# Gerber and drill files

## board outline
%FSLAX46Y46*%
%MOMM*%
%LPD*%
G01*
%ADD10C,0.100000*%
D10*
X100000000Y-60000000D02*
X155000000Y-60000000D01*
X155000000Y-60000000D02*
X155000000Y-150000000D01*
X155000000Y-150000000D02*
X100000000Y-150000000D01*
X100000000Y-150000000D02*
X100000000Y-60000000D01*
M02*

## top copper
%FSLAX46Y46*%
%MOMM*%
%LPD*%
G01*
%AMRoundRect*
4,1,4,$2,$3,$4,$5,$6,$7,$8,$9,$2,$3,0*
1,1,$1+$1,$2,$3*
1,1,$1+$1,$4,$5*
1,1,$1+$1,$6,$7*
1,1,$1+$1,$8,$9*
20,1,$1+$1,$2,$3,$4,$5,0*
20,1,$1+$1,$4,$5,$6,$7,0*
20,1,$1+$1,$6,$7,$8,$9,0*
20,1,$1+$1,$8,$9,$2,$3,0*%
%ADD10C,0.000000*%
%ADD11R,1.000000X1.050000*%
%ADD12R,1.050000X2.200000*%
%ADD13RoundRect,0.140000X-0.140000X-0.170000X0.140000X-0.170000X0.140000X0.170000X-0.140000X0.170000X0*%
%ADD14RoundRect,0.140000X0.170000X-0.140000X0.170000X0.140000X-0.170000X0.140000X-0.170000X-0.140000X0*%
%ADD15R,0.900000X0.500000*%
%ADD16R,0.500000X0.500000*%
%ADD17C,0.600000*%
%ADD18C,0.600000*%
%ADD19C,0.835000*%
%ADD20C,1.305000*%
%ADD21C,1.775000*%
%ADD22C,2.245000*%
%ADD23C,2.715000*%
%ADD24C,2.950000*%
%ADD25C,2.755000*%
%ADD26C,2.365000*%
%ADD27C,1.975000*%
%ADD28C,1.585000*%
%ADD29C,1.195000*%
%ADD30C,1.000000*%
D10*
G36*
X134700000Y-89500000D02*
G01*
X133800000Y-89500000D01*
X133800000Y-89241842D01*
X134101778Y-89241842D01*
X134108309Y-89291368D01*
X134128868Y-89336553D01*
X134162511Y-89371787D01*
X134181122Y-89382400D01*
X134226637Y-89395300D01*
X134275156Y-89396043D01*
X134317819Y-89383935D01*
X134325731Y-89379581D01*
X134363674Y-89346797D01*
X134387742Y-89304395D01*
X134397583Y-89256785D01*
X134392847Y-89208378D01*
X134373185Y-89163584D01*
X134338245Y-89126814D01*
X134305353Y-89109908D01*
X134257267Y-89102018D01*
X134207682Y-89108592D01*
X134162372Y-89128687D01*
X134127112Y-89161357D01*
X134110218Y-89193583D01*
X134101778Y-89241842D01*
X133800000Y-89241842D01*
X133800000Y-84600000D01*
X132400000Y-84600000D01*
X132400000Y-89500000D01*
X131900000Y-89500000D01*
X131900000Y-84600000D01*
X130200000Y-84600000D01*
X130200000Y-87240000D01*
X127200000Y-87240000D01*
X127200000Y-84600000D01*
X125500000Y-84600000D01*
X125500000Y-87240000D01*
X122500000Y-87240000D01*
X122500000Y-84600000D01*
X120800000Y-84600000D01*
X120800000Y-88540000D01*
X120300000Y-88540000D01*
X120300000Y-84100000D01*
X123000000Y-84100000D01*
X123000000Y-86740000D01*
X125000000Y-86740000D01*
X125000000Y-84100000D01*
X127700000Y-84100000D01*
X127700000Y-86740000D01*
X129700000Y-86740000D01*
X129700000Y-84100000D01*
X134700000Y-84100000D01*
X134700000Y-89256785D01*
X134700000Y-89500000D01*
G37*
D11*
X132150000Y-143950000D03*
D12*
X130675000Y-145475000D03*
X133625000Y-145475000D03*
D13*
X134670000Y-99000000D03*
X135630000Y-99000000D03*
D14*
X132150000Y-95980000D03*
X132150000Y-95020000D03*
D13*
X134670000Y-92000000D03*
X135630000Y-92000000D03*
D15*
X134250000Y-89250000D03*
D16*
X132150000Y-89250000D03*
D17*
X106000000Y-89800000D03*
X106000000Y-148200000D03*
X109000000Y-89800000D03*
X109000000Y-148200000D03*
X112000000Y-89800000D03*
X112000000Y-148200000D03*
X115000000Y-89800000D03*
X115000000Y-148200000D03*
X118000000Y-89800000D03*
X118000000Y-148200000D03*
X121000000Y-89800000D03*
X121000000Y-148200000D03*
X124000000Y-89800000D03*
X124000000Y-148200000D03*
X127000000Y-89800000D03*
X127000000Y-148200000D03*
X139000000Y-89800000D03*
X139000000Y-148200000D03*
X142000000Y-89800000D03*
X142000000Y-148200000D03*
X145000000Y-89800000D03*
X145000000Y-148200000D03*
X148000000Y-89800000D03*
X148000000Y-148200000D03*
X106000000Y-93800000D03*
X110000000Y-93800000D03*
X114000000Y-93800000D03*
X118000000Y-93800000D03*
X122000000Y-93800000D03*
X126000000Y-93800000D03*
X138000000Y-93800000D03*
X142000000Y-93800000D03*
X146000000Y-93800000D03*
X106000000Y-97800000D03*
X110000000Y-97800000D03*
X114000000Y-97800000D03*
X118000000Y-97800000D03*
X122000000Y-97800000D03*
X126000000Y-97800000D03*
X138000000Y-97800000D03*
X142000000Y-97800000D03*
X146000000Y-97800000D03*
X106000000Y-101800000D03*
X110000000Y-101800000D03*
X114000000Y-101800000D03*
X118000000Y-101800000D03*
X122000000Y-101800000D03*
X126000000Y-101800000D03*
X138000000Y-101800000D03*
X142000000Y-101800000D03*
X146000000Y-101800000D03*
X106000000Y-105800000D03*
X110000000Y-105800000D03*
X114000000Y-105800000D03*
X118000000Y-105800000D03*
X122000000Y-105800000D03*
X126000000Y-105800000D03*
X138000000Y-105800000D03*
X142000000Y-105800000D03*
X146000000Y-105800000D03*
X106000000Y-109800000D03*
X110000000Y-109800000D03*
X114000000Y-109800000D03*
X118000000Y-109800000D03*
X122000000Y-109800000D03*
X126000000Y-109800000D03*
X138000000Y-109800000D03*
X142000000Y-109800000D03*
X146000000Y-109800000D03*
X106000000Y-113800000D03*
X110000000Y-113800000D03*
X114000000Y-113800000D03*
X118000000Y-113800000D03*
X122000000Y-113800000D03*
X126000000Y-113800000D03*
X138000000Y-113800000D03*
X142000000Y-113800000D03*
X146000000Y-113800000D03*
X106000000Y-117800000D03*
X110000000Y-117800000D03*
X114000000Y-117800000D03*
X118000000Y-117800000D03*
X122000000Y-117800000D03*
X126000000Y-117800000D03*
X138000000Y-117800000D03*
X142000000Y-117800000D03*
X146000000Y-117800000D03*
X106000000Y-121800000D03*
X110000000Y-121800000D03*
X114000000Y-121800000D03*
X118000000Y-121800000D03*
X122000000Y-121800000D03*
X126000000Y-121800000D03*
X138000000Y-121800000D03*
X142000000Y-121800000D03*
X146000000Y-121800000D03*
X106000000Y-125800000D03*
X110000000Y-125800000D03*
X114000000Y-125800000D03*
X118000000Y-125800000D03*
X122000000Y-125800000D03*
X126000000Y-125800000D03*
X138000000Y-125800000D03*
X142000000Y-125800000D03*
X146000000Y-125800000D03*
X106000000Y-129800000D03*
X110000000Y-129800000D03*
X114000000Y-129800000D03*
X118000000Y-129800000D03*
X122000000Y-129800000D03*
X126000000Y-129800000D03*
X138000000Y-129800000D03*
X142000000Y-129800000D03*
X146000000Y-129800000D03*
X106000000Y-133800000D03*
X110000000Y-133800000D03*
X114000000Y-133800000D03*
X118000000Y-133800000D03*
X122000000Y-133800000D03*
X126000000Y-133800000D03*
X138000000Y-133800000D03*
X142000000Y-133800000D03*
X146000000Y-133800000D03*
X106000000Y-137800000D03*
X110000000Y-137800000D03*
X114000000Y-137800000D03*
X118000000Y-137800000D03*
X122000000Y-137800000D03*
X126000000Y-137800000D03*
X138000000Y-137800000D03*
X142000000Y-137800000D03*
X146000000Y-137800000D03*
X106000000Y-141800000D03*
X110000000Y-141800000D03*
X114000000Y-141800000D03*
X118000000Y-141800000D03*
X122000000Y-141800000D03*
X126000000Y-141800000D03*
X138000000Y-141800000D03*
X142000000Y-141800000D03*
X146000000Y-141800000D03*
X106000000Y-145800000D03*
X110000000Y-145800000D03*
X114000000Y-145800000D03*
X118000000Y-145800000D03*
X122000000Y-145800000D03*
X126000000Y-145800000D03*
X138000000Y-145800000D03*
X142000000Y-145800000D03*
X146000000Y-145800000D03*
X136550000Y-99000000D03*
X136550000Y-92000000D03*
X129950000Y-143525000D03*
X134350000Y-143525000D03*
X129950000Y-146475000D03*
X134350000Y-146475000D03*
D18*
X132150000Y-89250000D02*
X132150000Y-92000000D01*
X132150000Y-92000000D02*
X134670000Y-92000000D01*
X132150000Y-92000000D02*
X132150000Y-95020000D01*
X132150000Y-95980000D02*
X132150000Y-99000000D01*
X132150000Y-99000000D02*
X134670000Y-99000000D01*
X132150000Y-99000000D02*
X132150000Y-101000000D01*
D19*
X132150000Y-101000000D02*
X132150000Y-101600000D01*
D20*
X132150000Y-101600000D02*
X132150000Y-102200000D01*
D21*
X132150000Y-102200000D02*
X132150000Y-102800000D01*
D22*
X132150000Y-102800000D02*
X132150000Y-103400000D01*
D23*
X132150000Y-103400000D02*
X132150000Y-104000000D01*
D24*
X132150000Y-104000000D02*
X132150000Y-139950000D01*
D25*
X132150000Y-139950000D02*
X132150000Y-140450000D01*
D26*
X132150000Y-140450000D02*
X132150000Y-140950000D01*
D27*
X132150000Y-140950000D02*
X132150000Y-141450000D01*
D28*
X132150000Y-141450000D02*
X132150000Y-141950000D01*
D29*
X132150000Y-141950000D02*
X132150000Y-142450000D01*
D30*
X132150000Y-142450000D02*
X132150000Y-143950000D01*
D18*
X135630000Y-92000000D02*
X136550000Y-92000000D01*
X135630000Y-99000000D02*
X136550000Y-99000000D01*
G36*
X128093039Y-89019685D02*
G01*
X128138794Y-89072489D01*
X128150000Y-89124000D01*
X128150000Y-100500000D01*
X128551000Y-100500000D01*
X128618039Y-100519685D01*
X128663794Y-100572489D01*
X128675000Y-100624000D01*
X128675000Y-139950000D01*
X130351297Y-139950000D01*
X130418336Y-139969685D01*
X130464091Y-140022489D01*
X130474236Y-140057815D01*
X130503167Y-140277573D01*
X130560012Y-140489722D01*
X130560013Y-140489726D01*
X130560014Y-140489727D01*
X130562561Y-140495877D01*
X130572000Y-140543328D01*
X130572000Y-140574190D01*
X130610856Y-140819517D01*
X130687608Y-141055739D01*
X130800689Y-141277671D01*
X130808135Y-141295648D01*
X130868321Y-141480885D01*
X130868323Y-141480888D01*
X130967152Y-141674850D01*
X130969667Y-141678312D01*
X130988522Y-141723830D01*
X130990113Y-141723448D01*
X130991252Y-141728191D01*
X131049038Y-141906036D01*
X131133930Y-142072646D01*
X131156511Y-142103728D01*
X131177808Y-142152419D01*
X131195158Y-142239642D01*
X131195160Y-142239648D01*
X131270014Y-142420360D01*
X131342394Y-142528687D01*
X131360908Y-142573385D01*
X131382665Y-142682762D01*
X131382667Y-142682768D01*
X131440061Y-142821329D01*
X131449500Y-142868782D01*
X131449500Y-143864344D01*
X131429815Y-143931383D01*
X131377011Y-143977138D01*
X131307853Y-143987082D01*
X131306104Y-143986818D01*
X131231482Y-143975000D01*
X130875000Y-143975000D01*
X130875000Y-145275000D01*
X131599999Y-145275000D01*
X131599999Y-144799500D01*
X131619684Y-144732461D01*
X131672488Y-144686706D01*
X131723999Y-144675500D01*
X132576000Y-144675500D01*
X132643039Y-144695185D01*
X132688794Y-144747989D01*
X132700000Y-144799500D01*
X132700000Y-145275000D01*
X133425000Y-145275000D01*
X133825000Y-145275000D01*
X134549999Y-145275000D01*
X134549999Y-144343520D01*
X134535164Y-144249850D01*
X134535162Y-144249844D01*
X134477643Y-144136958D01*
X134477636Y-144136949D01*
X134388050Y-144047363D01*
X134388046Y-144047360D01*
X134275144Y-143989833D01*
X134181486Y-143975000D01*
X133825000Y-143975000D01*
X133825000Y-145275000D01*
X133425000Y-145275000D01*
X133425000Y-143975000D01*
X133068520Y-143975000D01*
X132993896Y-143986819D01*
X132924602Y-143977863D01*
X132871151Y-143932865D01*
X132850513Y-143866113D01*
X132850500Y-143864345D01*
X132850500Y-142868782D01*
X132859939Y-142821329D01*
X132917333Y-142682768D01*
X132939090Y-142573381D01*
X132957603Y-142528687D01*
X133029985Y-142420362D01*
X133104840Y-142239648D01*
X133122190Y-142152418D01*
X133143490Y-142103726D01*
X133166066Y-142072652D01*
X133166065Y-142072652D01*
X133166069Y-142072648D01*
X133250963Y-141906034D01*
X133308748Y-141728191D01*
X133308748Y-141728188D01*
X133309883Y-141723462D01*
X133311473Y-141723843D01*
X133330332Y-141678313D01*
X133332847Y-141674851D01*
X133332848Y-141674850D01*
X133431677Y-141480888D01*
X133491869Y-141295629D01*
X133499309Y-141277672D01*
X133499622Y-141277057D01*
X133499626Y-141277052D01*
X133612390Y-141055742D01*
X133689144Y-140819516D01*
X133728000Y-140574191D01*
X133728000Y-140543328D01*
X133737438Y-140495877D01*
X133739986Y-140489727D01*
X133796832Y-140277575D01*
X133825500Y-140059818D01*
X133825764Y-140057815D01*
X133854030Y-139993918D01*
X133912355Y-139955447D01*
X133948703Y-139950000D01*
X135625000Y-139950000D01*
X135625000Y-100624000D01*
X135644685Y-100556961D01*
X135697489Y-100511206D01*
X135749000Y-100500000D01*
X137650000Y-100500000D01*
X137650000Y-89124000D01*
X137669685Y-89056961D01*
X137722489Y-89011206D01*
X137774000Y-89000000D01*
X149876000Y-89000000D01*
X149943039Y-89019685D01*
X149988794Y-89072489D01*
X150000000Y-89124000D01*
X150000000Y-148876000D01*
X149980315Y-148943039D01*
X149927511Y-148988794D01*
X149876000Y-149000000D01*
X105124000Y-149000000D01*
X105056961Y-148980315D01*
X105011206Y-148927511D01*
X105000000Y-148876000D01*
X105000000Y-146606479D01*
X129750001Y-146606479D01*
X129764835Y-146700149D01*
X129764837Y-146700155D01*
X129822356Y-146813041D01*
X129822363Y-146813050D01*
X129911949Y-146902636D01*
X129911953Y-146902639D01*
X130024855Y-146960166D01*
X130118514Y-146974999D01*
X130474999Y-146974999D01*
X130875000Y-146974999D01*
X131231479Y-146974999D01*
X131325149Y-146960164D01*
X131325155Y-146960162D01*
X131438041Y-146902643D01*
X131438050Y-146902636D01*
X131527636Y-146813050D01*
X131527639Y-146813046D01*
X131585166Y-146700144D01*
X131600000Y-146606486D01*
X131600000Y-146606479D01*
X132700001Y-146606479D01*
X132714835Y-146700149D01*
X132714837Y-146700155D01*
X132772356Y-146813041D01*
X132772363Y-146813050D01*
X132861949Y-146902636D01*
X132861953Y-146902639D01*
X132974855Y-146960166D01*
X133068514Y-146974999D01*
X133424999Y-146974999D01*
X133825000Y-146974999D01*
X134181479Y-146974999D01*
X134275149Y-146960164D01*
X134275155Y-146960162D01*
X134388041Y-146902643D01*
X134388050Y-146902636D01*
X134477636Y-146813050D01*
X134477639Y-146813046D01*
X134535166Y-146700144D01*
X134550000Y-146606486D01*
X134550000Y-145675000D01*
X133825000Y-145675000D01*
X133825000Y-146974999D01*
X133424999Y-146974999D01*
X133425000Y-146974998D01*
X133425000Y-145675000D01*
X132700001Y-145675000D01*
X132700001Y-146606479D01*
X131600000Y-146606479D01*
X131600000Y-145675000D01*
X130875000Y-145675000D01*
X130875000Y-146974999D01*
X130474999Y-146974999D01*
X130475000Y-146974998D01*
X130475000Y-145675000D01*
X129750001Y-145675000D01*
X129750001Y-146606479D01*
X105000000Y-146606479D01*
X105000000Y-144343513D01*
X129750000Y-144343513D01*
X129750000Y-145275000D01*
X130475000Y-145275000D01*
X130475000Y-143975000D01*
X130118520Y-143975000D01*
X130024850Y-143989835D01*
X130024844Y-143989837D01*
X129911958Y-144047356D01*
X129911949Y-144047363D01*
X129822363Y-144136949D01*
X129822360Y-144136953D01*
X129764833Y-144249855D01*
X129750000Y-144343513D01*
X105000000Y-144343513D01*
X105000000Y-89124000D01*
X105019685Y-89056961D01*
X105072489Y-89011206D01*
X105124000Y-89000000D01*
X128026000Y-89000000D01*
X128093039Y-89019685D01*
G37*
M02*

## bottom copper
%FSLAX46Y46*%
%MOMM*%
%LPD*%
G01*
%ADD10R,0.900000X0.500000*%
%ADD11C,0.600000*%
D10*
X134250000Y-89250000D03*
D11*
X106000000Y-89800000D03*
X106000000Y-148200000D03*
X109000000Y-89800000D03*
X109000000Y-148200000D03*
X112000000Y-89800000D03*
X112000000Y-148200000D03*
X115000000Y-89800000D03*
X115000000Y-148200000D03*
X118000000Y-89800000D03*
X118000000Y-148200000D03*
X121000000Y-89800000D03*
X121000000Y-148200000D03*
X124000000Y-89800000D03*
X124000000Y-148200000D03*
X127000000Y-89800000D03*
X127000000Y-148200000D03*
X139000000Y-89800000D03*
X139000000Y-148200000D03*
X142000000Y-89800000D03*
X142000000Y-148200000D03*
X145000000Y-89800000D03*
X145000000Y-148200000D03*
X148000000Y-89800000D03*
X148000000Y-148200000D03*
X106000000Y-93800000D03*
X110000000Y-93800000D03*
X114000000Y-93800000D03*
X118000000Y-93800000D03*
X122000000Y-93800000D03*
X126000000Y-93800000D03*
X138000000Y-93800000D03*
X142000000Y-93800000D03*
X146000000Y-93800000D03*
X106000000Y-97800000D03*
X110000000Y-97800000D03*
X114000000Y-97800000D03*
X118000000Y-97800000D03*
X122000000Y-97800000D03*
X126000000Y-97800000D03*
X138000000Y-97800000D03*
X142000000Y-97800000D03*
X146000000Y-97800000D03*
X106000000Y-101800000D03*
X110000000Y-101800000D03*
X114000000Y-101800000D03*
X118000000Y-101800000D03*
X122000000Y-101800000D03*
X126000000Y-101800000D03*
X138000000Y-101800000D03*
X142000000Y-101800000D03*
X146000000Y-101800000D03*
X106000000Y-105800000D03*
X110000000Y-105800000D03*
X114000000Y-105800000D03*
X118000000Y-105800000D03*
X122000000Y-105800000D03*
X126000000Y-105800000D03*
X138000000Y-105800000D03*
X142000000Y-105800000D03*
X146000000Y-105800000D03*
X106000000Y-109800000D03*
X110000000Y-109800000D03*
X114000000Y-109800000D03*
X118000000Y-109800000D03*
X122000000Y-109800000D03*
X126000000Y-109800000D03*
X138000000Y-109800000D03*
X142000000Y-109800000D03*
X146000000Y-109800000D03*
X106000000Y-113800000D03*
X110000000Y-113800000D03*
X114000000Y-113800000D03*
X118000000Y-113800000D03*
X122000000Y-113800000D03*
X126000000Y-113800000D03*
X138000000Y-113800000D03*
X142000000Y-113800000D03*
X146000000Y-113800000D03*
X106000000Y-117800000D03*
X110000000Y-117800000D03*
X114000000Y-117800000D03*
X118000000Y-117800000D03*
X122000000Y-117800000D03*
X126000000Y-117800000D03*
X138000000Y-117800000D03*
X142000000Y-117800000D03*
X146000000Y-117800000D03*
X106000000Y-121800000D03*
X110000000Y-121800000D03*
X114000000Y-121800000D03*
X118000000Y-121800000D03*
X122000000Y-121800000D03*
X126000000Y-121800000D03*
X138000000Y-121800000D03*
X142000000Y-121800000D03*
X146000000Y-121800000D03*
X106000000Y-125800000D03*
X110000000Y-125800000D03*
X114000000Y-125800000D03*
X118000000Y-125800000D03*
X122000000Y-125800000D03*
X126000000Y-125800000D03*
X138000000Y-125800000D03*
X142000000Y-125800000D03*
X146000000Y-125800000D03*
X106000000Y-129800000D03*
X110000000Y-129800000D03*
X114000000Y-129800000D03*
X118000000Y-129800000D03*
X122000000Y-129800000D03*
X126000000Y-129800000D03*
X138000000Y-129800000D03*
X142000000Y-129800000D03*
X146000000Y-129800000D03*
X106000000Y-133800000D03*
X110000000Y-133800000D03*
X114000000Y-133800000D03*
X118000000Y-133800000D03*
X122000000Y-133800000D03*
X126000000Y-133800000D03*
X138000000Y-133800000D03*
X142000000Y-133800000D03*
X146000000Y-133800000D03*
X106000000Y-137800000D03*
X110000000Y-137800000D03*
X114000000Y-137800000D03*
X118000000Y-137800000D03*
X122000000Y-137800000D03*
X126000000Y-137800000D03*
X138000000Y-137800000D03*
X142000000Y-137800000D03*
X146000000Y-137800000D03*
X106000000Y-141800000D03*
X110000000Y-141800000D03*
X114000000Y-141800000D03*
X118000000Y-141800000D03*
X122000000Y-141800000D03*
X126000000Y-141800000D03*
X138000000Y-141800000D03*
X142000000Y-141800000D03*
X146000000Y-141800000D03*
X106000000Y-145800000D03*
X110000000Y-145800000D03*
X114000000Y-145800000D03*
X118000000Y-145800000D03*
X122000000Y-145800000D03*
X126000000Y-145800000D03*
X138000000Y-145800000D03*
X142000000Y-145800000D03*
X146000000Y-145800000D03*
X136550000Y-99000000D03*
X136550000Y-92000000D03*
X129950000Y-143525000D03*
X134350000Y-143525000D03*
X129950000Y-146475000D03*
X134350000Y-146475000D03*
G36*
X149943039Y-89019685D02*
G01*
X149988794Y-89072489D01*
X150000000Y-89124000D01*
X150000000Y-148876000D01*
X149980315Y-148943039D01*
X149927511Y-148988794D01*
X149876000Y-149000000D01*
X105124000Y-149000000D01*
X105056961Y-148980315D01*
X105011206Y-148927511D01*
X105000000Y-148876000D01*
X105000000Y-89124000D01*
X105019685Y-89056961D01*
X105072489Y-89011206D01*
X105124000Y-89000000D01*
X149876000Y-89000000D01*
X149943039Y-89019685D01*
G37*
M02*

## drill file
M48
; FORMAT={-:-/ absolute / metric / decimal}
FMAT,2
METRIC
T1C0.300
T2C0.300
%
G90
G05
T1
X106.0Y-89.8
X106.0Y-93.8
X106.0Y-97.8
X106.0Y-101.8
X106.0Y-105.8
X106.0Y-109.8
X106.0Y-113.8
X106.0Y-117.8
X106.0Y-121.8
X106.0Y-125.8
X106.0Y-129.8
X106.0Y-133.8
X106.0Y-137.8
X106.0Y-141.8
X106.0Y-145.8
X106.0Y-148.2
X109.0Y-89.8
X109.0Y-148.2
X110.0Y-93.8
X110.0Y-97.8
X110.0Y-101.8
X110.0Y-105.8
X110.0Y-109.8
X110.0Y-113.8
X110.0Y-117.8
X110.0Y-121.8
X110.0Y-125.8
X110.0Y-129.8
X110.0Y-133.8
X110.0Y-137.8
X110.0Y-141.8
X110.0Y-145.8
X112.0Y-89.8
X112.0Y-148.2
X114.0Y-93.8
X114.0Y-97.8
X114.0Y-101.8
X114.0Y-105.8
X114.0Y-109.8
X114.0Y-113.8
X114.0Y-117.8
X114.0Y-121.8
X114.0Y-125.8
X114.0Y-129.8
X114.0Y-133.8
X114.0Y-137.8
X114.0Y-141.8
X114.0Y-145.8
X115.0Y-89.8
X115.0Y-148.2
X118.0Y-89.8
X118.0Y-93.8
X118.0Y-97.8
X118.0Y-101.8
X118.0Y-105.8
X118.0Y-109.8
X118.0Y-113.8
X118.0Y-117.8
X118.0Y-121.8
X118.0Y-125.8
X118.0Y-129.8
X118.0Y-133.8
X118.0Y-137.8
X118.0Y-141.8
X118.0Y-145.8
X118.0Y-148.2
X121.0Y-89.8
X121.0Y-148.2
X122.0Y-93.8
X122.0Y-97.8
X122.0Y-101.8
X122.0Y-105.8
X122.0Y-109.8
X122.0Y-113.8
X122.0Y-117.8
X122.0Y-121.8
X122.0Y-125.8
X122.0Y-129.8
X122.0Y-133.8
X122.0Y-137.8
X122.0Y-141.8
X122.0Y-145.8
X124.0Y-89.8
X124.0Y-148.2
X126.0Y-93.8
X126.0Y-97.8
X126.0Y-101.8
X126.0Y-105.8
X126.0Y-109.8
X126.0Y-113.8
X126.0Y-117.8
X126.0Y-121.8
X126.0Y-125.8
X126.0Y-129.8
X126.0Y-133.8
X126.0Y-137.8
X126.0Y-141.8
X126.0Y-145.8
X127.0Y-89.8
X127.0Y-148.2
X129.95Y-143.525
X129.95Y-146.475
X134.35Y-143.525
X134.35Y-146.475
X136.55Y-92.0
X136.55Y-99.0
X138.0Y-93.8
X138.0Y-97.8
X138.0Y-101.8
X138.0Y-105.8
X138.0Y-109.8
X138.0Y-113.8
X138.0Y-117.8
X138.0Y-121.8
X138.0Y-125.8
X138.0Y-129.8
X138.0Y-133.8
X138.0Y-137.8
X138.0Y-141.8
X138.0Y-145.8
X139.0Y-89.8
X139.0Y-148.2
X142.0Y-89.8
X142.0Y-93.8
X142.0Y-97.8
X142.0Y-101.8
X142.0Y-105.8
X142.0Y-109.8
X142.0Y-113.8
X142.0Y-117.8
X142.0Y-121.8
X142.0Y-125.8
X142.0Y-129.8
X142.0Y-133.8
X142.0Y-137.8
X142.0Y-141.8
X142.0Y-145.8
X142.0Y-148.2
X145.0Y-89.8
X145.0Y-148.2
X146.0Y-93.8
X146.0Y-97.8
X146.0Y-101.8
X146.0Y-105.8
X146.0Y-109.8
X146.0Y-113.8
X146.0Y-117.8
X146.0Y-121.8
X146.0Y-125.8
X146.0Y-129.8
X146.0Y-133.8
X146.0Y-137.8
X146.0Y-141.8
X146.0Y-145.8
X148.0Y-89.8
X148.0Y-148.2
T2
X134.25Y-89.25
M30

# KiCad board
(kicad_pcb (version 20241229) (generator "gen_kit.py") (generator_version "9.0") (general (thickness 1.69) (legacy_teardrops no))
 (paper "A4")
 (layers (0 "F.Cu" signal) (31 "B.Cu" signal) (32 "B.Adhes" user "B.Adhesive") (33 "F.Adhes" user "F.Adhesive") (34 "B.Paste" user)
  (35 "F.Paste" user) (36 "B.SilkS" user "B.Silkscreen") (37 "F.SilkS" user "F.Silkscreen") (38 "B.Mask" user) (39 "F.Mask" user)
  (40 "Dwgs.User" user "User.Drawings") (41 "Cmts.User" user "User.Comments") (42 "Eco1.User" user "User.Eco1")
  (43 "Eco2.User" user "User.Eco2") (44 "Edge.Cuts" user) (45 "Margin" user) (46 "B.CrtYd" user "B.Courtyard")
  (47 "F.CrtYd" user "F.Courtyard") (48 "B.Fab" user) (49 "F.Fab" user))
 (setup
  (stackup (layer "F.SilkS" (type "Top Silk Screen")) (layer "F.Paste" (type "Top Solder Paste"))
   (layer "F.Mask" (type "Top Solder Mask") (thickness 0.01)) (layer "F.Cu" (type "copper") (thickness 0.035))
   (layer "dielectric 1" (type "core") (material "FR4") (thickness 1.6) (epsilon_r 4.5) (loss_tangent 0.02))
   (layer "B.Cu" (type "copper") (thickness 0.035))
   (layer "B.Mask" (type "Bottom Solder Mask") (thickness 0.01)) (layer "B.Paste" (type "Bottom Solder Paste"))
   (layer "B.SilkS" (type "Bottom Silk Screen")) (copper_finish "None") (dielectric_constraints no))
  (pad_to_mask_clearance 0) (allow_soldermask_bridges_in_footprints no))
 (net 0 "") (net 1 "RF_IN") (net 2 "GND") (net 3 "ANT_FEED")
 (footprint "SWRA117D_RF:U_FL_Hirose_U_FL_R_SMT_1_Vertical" (layer "F.Cu") (at 132.15 145 270)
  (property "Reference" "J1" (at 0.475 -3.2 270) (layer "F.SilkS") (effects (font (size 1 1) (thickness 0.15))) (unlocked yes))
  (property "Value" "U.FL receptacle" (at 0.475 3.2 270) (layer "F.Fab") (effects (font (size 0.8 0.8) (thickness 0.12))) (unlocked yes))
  (pad "1" smd rect (at -1.05 0 270) (size 1.05 1) (layers "F.Cu" "F.Paste" "F.Mask") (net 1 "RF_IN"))
  (pad "2" smd rect (at 0.475 1.475 270) (size 2.2 1.05) (layers "F.Cu" "F.Paste" "F.Mask") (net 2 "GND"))
  (pad "2" smd rect (at 0.475 -1.475 270) (size 2.2 1.05) (layers "F.Cu" "F.Paste" "F.Mask") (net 2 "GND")))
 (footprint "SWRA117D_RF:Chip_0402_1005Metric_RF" (layer "F.Cu") (at 135.15 99)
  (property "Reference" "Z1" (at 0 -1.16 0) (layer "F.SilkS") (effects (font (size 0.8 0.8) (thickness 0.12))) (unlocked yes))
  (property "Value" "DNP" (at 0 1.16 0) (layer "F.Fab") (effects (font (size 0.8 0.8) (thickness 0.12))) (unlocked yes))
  (pad "1" smd roundrect (at -0.48 0) (size 0.56 0.62) (layers "F.Cu" "F.Paste" "F.Mask") (roundrect_rratio 0.25) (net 1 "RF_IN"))
  (pad "2" smd roundrect (at 0.48 0) (size 0.56 0.62) (layers "F.Cu" "F.Paste" "F.Mask") (roundrect_rratio 0.25) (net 2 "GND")))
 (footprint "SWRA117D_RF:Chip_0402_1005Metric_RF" (layer "F.Cu") (at 132.15 95.5 90)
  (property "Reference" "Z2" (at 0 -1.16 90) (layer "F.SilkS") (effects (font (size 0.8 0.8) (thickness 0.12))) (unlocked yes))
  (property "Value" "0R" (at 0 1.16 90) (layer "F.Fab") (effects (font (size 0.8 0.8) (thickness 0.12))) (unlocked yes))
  (pad "1" smd roundrect (at -0.48 0 90) (size 0.56 0.62) (layers "F.Cu" "F.Paste" "F.Mask") (roundrect_rratio 0.25) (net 1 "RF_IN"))
  (pad "2" smd roundrect (at 0.48 0 90) (size 0.56 0.62) (layers "F.Cu" "F.Paste" "F.Mask") (roundrect_rratio 0.25) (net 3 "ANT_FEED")))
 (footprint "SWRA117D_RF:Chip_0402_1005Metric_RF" (layer "F.Cu") (at 135.15 92)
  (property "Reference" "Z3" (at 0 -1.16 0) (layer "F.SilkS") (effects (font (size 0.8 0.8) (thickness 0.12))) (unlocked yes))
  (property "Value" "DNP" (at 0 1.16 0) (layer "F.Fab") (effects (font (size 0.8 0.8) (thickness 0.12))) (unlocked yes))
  (pad "1" smd roundrect (at -0.48 0) (size 0.56 0.62) (layers "F.Cu" "F.Paste" "F.Mask") (roundrect_rratio 0.25) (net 3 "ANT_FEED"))
  (pad "2" smd roundrect (at 0.48 0) (size 0.56 0.62) (layers "F.Cu" "F.Paste" "F.Mask") (roundrect_rratio 0.25) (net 2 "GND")))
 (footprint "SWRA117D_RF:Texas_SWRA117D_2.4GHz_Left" (layer "F.Cu") (at 132.15 89.25)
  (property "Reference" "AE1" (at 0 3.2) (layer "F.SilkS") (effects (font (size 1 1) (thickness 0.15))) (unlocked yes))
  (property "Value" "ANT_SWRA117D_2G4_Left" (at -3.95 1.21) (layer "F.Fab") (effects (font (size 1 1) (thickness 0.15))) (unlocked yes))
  (fp_poly
   (pts (xy -2.45 -2.51) (xy -4.45 -2.51) (xy -4.45 -5.15) (xy -7.15 -5.15) (xy -7.15 -2.51) (xy -9.15 -2.51) (xy -9.15 -5.15)
    (xy -11.85 -5.15) (xy -11.85 -0.71) (xy -11.35 -0.71) (xy -11.35 -4.65) (xy -9.65 -4.65) (xy -9.65 -2.01) (xy -6.65 -2.01)
    (xy -6.65 -4.65) (xy -4.95 -4.65) (xy -4.95 -2.01) (xy -1.95 -2.01) (xy -1.95 -4.65) (xy -0.25 -4.65) (xy -0.25 0.25) (xy 0.25 0.25)
    (xy 0.25 -4.65) (xy 1.65 -4.65) (xy 1.65 0.25) (xy 2.55 0.25) (xy 2.55 0.006785) (xy 2.247583 0.006785) (xy 2.237742 0.054395)
    (xy 2.213674 0.096797) (xy 2.175731 0.129581) (xy 2.167819 0.133935) (xy 2.125156 0.146043) (xy 2.076637 0.1453) (xy 2.031122 0.1324)
    (xy 2.012511 0.121787) (xy 1.978868 0.086553) (xy 1.958309 0.041368) (xy 1.951778 -0.008158) (xy 1.960218 -0.056417)
    (xy 1.977112 -0.088643) (xy 2.012372 -0.121313) (xy 2.057682 -0.141408) (xy 2.107267 -0.147982) (xy 2.155353 -0.140092)
    (xy 2.188245 -0.123186) (xy 2.223185 -0.086416) (xy 2.242847 -0.041622) (xy 2.247583 0.006785) (xy 2.55 0.006785) (xy 2.55 -5.15)
    (xy -2.45 -5.15) (xy -2.45 -2.51))
   (stroke (width 0) (type solid)) (fill yes) (layer "F.Cu"))
  (pad "2" thru_hole rect (at 2.1 0) (size 0.9 0.5) (drill 0.3) (layers "*.Cu") (zone_connect 2) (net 2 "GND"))
  (pad "1" smd rect (at 0 0) (size 0.5 0.5) (layers "F.Cu") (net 3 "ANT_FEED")))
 (gr_line (start 100 60) (end 155 60) (stroke (width 0.1) (type solid)) (layer "Edge.Cuts"))
 (gr_line (start 155 60) (end 155 150) (stroke (width 0.1) (type solid)) (layer "Edge.Cuts"))
 (gr_line (start 155 150) (end 100 150) (stroke (width 0.1) (type solid)) (layer "Edge.Cuts"))
 (gr_line (start 100 150) (end 100 60) (stroke (width 0.1) (type solid)) (layer "Edge.Cuts"))
 (segment (start 132.15 89.25) (end 132.15 92) (width 0.6) (layer "F.Cu") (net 3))
 (segment (start 132.15 92) (end 134.67 92) (width 0.6) (layer "F.Cu") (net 3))
 (segment (start 132.15 92) (end 132.15 95.02) (width 0.6) (layer "F.Cu") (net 3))
 (segment (start 132.15 95.98) (end 132.15 99) (width 0.6) (layer "F.Cu") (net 1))
 (segment (start 132.15 99) (end 134.67 99) (width 0.6) (layer "F.Cu") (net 1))
 (segment (start 132.15 99) (end 132.15 101) (width 0.6) (layer "F.Cu") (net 1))
 (segment (start 132.15 101) (end 132.15 101.6) (width 0.835) (layer "F.Cu") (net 1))
 (segment (start 132.15 101.6) (end 132.15 102.2) (width 1.305) (layer "F.Cu") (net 1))
 (segment (start 132.15 102.2) (end 132.15 102.8) (width 1.775) (layer "F.Cu") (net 1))
 (segment (start 132.15 102.8) (end 132.15 103.4) (width 2.245) (layer "F.Cu") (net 1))
 (segment (start 132.15 103.4) (end 132.15 104) (width 2.715) (layer "F.Cu") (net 1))
 (segment (start 132.15 104) (end 132.15 139.95) (width 2.95) (layer "F.Cu") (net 1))
 (segment (start 132.15 139.95) (end 132.15 140.45) (width 2.755) (layer "F.Cu") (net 1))
 (segment (start 132.15 140.45) (end 132.15 140.95) (width 2.365) (layer "F.Cu") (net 1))
 (segment (start 132.15 140.95) (end 132.15 141.45) (width 1.975) (layer "F.Cu") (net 1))
 (segment (start 132.15 141.45) (end 132.15 141.95) (width 1.585) (layer "F.Cu") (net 1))
 (segment (start 132.15 141.95) (end 132.15 142.45) (width 1.195) (layer "F.Cu") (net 1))
 (segment (start 132.15 142.45) (end 132.15 143.95) (width 1) (layer "F.Cu") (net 1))
 (segment (start 135.63 92) (end 136.55 92) (width 0.6) (layer "F.Cu") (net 2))
 (segment (start 135.63 99) (end 136.55 99) (width 0.6) (layer "F.Cu") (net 2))
 (via (at 106 89.8) (size 0.6) (drill 0.3) (layers "F.Cu" "B.Cu") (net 2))
 (via (at 106 148.2) (size 0.6) (drill 0.3) (layers "F.Cu" "B.Cu") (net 2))
 (via (at 109 89.8) (size 0.6) (drill 0.3) (layers "F.Cu" "B.Cu") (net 2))
 (via (at 109 148.2) (size 0.6) (drill 0.3) (layers "F.Cu" "B.Cu") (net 2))
 (via (at 112 89.8) (size 0.6) (drill 0.3) (layers "F.Cu" "B.Cu") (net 2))
 (via (at 112 148.2) (size 0.6) (drill 0.3) (layers "F.Cu" "B.Cu") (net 2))
 (via (at 115 89.8) (size 0.6) (drill 0.3) (layers "F.Cu" "B.Cu") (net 2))
 (via (at 115 148.2) (size 0.6) (drill 0.3) (layers "F.Cu" "B.Cu") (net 2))
 (via (at 118 89.8) (size 0.6) (drill 0.3) (layers "F.Cu" "B.Cu") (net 2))
 (via (at 118 148.2) (size 0.6) (drill 0.3) (layers "F.Cu" "B.Cu") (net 2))
 (via (at 121 89.8) (size 0.6) (drill 0.3) (layers "F.Cu" "B.Cu") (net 2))
 (via (at 121 148.2) (size 0.6) (drill 0.3) (layers "F.Cu" "B.Cu") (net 2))
 (via (at 124 89.8) (size 0.6) (drill 0.3) (layers "F.Cu" "B.Cu") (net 2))
 (via (at 124 148.2) (size 0.6) (drill 0.3) (layers "F.Cu" "B.Cu") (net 2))
 (via (at 127 89.8) (size 0.6) (drill 0.3) (layers "F.Cu" "B.Cu") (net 2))
 (via (at 127 148.2) (size 0.6) (drill 0.3) (layers "F.Cu" "B.Cu") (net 2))
 (via (at 139 89.8) (size 0.6) (drill 0.3) (layers "F.Cu" "B.Cu") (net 2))
 (via (at 139 148.2) (size 0.6) (drill 0.3) (layers "F.Cu" "B.Cu") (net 2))
 (via (at 142 89.8) (size 0.6) (drill 0.3) (layers "F.Cu" "B.Cu") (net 2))
 (via (at 142 148.2) (size 0.6) (drill 0.3) (layers "F.Cu" "B.Cu") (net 2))
 (via (at 145 89.8) (size 0.6) (drill 0.3) (layers "F.Cu" "B.Cu") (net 2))
 (via (at 145 148.2) (size 0.6) (drill 0.3) (layers "F.Cu" "B.Cu") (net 2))
 (via (at 148 89.8) (size 0.6) (drill 0.3) (layers "F.Cu" "B.Cu") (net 2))
 (via (at 148 148.2) (size 0.6) (drill 0.3) (layers "F.Cu" "B.Cu") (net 2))
 (via (at 106 93.8) (size 0.6) (drill 0.3) (layers "F.Cu" "B.Cu") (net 2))
 (via (at 110 93.8) (size 0.6) (drill 0.3) (layers "F.Cu" "B.Cu") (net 2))
 (via (at 114 93.8) (size 0.6) (drill 0.3) (layers "F.Cu" "B.Cu") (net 2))
 (via (at 118 93.8) (size 0.6) (drill 0.3) (layers "F.Cu" "B.Cu") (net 2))
 (via (at 122 93.8) (size 0.6) (drill 0.3) (layers "F.Cu" "B.Cu") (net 2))
 (via (at 126 93.8) (size 0.6) (drill 0.3) (layers "F.Cu" "B.Cu") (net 2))
 (via (at 138 93.8) (size 0.6) (drill 0.3) (layers "F.Cu" "B.Cu") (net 2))
 (via (at 142 93.8) (size 0.6) (drill 0.3) (layers "F.Cu" "B.Cu") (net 2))
 (via (at 146 93.8) (size 0.6) (drill 0.3) (layers "F.Cu" "B.Cu") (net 2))
 (via (at 106 97.8) (size 0.6) (drill 0.3) (layers "F.Cu" "B.Cu") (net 2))
 (via (at 110 97.8) (size 0.6) (drill 0.3) (layers "F.Cu" "B.Cu") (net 2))
 (via (at 114 97.8) (size 0.6) (drill 0.3) (layers "F.Cu" "B.Cu") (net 2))
 (via (at 118 97.8) (size 0.6) (drill 0.3) (layers "F.Cu" "B.Cu") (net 2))
 (via (at 122 97.8) (size 0.6) (drill 0.3) (layers "F.Cu" "B.Cu") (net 2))
 (via (at 126 97.8) (size 0.6) (drill 0.3) (layers "F.Cu" "B.Cu") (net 2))
 (via (at 138 97.8) (size 0.6) (drill 0.3) (layers "F.Cu" "B.Cu") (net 2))
 (via (at 142 97.8) (size 0.6) (drill 0.3) (layers "F.Cu" "B.Cu") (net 2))
 (via (at 146 97.8) (size 0.6) (drill 0.3) (layers "F.Cu" "B.Cu") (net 2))
 (via (at 106 101.8) (size 0.6) (drill 0.3) (layers "F.Cu" "B.Cu") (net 2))
 (via (at 110 101.8) (size 0.6) (drill 0.3) (layers "F.Cu" "B.Cu") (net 2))
 (via (at 114 101.8) (size 0.6) (drill 0.3) (layers "F.Cu" "B.Cu") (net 2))
 (via (at 118 101.8) (size 0.6) (drill 0.3) (layers "F.Cu" "B.Cu") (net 2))
 (via (at 122 101.8) (size 0.6) (drill 0.3) (layers "F.Cu" "B.Cu") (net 2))
 (via (at 126 101.8) (size 0.6) (drill 0.3) (layers "F.Cu" "B.Cu") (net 2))
 (via (at 138 101.8) (size 0.6) (drill 0.3) (layers "F.Cu" "B.Cu") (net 2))
 (via (at 142 101.8) (size 0.6) (drill 0.3) (layers "F.Cu" "B.Cu") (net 2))
 (via (at 146 101.8) (size 0.6) (drill 0.3) (layers "F.Cu" "B.Cu") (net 2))
 (via (at 106 105.8) (size 0.6) (drill 0.3) (layers "F.Cu" "B.Cu") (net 2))
 (via (at 110 105.8) (size 0.6) (drill 0.3) (layers "F.Cu" "B.Cu") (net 2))
 (via (at 114 105.8) (size 0.6) (drill 0.3) (layers "F.Cu" "B.Cu") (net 2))
 (via (at 118 105.8) (size 0.6) (drill 0.3) (layers "F.Cu" "B.Cu") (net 2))
 (via (at 122 105.8) (size 0.6) (drill 0.3) (layers "F.Cu" "B.Cu") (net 2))
 (via (at 126 105.8) (size 0.6) (drill 0.3) (layers "F.Cu" "B.Cu") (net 2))
 (via (at 138 105.8) (size 0.6) (drill 0.3) (layers "F.Cu" "B.Cu") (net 2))
 (via (at 142 105.8) (size 0.6) (drill 0.3) (layers "F.Cu" "B.Cu") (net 2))
 (via (at 146 105.8) (size 0.6) (drill 0.3) (layers "F.Cu" "B.Cu") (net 2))
 (via (at 106 109.8) (size 0.6) (drill 0.3) (layers "F.Cu" "B.Cu") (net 2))
 (via (at 110 109.8) (size 0.6) (drill 0.3) (layers "F.Cu" "B.Cu") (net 2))
 (via (at 114 109.8) (size 0.6) (drill 0.3) (layers "F.Cu" "B.Cu") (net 2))
 (via (at 118 109.8) (size 0.6) (drill 0.3) (layers "F.Cu" "B.Cu") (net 2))
 (via (at 122 109.8) (size 0.6) (drill 0.3) (layers "F.Cu" "B.Cu") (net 2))
 (via (at 126 109.8) (size 0.6) (drill 0.3) (layers "F.Cu" "B.Cu") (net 2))
 (via (at 138 109.8) (size 0.6) (drill 0.3) (layers "F.Cu" "B.Cu") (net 2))
 (via (at 142 109.8) (size 0.6) (drill 0.3) (layers "F.Cu" "B.Cu") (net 2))
 (via (at 146 109.8) (size 0.6) (drill 0.3) (layers "F.Cu" "B.Cu") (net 2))
 (via (at 106 113.8) (size 0.6) (drill 0.3) (layers "F.Cu" "B.Cu") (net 2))
 (via (at 110 113.8) (size 0.6) (drill 0.3) (layers "F.Cu" "B.Cu") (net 2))
 (via (at 114 113.8) (size 0.6) (drill 0.3) (layers "F.Cu" "B.Cu") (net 2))
 (via (at 118 113.8) (size 0.6) (drill 0.3) (layers "F.Cu" "B.Cu") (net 2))
 (via (at 122 113.8) (size 0.6) (drill 0.3) (layers "F.Cu" "B.Cu") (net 2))
 (via (at 126 113.8) (size 0.6) (drill 0.3) (layers "F.Cu" "B.Cu") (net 2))
 (via (at 138 113.8) (size 0.6) (drill 0.3) (layers "F.Cu" "B.Cu") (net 2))
 (via (at 142 113.8) (size 0.6) (drill 0.3) (layers "F.Cu" "B.Cu") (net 2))
 (via (at 146 113.8) (size 0.6) (drill 0.3) (layers "F.Cu" "B.Cu") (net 2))
 (via (at 106 117.8) (size 0.6) (drill 0.3) (layers "F.Cu" "B.Cu") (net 2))
 (via (at 110 117.8) (size 0.6) (drill 0.3) (layers "F.Cu" "B.Cu") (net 2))
 (via (at 114 117.8) (size 0.6) (drill 0.3) (layers "F.Cu" "B.Cu") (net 2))
 (via (at 118 117.8) (size 0.6) (drill 0.3) (layers "F.Cu" "B.Cu") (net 2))
 (via (at 122 117.8) (size 0.6) (drill 0.3) (layers "F.Cu" "B.Cu") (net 2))
 (via (at 126 117.8) (size 0.6) (drill 0.3) (layers "F.Cu" "B.Cu") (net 2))
 (via (at 138 117.8) (size 0.6) (drill 0.3) (layers "F.Cu" "B.Cu") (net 2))
 (via (at 142 117.8) (size 0.6) (drill 0.3) (layers "F.Cu" "B.Cu") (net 2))
 (via (at 146 117.8) (size 0.6) (drill 0.3) (layers "F.Cu" "B.Cu") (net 2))
 (via (at 106 121.8) (size 0.6) (drill 0.3) (layers "F.Cu" "B.Cu") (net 2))
 (via (at 110 121.8) (size 0.6) (drill 0.3) (layers "F.Cu" "B.Cu") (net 2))
 (via (at 114 121.8) (size 0.6) (drill 0.3) (layers "F.Cu" "B.Cu") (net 2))
 (via (at 118 121.8) (size 0.6) (drill 0.3) (layers "F.Cu" "B.Cu") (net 2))
 (via (at 122 121.8) (size 0.6) (drill 0.3) (layers "F.Cu" "B.Cu") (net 2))
 (via (at 126 121.8) (size 0.6) (drill 0.3) (layers "F.Cu" "B.Cu") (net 2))
 (via (at 138 121.8) (size 0.6) (drill 0.3) (layers "F.Cu" "B.Cu") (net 2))
 (via (at 142 121.8) (size 0.6) (drill 0.3) (layers "F.Cu" "B.Cu") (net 2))
 (via (at 146 121.8) (size 0.6) (drill 0.3) (layers "F.Cu" "B.Cu") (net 2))
 (via (at 106 125.8) (size 0.6) (drill 0.3) (layers "F.Cu" "B.Cu") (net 2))
 (via (at 110 125.8) (size 0.6) (drill 0.3) (layers "F.Cu" "B.Cu") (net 2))
 (via (at 114 125.8) (size 0.6) (drill 0.3) (layers "F.Cu" "B.Cu") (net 2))
 (via (at 118 125.8) (size 0.6) (drill 0.3) (layers "F.Cu" "B.Cu") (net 2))
 (via (at 122 125.8) (size 0.6) (drill 0.3) (layers "F.Cu" "B.Cu") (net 2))
 (via (at 126 125.8) (size 0.6) (drill 0.3) (layers "F.Cu" "B.Cu") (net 2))
 (via (at 138 125.8) (size 0.6) (drill 0.3) (layers "F.Cu" "B.Cu") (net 2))
 (via (at 142 125.8) (size 0.6) (drill 0.3) (layers "F.Cu" "B.Cu") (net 2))
 (via (at 146 125.8) (size 0.6) (drill 0.3) (layers "F.Cu" "B.Cu") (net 2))
 (via (at 106 129.8) (size 0.6) (drill 0.3) (layers "F.Cu" "B.Cu") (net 2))
 (via (at 110 129.8) (size 0.6) (drill 0.3) (layers "F.Cu" "B.Cu") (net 2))
 (via (at 114 129.8) (size 0.6) (drill 0.3) (layers "F.Cu" "B.Cu") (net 2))
 (via (at 118 129.8) (size 0.6) (drill 0.3) (layers "F.Cu" "B.Cu") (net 2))
 (via (at 122 129.8) (size 0.6) (drill 0.3) (layers "F.Cu" "B.Cu") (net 2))
 (via (at 126 129.8) (size 0.6) (drill 0.3) (layers "F.Cu" "B.Cu") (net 2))
 (via (at 138 129.8) (size 0.6) (drill 0.3) (layers "F.Cu" "B.Cu") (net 2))
 (via (at 142 129.8) (size 0.6) (drill 0.3) (layers "F.Cu" "B.Cu") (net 2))
 (via (at 146 129.8) (size 0.6) (drill 0.3) (layers "F.Cu" "B.Cu") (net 2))
 (via (at 106 133.8) (size 0.6) (drill 0.3) (layers "F.Cu" "B.Cu") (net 2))
 (via (at 110 133.8) (size 0.6) (drill 0.3) (layers "F.Cu" "B.Cu") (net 2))
 (via (at 114 133.8) (size 0.6) (drill 0.3) (layers "F.Cu" "B.Cu") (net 2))
 (via (at 118 133.8) (size 0.6) (drill 0.3) (layers "F.Cu" "B.Cu") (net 2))
 (via (at 122 133.8) (size 0.6) (drill 0.3) (layers "F.Cu" "B.Cu") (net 2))
 (via (at 126 133.8) (size 0.6) (drill 0.3) (layers "F.Cu" "B.Cu") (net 2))
 (via (at 138 133.8) (size 0.6) (drill 0.3) (layers "F.Cu" "B.Cu") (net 2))
 (via (at 142 133.8) (size 0.6) (drill 0.3) (layers "F.Cu" "B.Cu") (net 2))
 (via (at 146 133.8) (size 0.6) (drill 0.3) (layers "F.Cu" "B.Cu") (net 2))
 (via (at 106 137.8) (size 0.6) (drill 0.3) (layers "F.Cu" "B.Cu") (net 2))
 (via (at 110 137.8) (size 0.6) (drill 0.3) (layers "F.Cu" "B.Cu") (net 2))
 (via (at 114 137.8) (size 0.6) (drill 0.3) (layers "F.Cu" "B.Cu") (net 2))
 (via (at 118 137.8) (size 0.6) (drill 0.3) (layers "F.Cu" "B.Cu") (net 2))
 (via (at 122 137.8) (size 0.6) (drill 0.3) (layers "F.Cu" "B.Cu") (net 2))
 (via (at 126 137.8) (size 0.6) (drill 0.3) (layers "F.Cu" "B.Cu") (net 2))
 (via (at 138 137.8) (size 0.6) (drill 0.3) (layers "F.Cu" "B.Cu") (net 2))
 (via (at 142 137.8) (size 0.6) (drill 0.3) (layers "F.Cu" "B.Cu") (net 2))
 (via (at 146 137.8) (size 0.6) (drill 0.3) (layers "F.Cu" "B.Cu") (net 2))
 (via (at 106 141.8) (size 0.6) (drill 0.3) (layers "F.Cu" "B.Cu") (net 2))
 (via (at 110 141.8) (size 0.6) (drill 0.3) (layers "F.Cu" "B.Cu") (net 2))
 (via (at 114 141.8) (size 0.6) (drill 0.3) (layers "F.Cu" "B.Cu") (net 2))
 (via (at 118 141.8) (size 0.6) (drill 0.3) (layers "F.Cu" "B.Cu") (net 2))
 (via (at 122 141.8) (size 0.6) (drill 0.3) (layers "F.Cu" "B.Cu") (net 2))
 (via (at 126 141.8) (size 0.6) (drill 0.3) (layers "F.Cu" "B.Cu") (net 2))
 (via (at 138 141.8) (size 0.6) (drill 0.3) (layers "F.Cu" "B.Cu") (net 2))
 (via (at 142 141.8) (size 0.6) (drill 0.3) (layers "F.Cu" "B.Cu") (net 2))
 (via (at 146 141.8) (size 0.6) (drill 0.3) (layers "F.Cu" "B.Cu") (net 2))
 (via (at 106 145.8) (size 0.6) (drill 0.3) (layers "F.Cu" "B.Cu") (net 2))
 (via (at 110 145.8) (size 0.6) (drill 0.3) (layers "F.Cu" "B.Cu") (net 2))
 (via (at 114 145.8) (size 0.6) (drill 0.3) (layers "F.Cu" "B.Cu") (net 2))
 (via (at 118 145.8) (size 0.6) (drill 0.3) (layers "F.Cu" "B.Cu") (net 2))
 (via (at 122 145.8) (size 0.6) (drill 0.3) (layers "F.Cu" "B.Cu") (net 2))
 (via (at 126 145.8) (size 0.6) (drill 0.3) (layers "F.Cu" "B.Cu") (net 2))
 (via (at 138 145.8) (size 0.6) (drill 0.3) (layers "F.Cu" "B.Cu") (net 2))
 (via (at 142 145.8) (size 0.6) (drill 0.3) (layers "F.Cu" "B.Cu") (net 2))
 (via (at 146 145.8) (size 0.6) (drill 0.3) (layers "F.Cu" "B.Cu") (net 2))
 (via (at 136.55 99) (size 0.6) (drill 0.3) (layers "F.Cu" "B.Cu") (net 2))
 (via (at 136.55 92) (size 0.6) (drill 0.3) (layers "F.Cu" "B.Cu") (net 2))
 (via (at 129.95 143.525) (size 0.6) (drill 0.3) (layers "F.Cu" "B.Cu") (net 2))
 (via (at 134.35 143.525) (size 0.6) (drill 0.3) (layers "F.Cu" "B.Cu") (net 2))
 (via (at 129.95 146.475) (size 0.6) (drill 0.3) (layers "F.Cu" "B.Cu") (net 2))
 (via (at 134.35 146.475) (size 0.6) (drill 0.3) (layers "F.Cu" "B.Cu") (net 2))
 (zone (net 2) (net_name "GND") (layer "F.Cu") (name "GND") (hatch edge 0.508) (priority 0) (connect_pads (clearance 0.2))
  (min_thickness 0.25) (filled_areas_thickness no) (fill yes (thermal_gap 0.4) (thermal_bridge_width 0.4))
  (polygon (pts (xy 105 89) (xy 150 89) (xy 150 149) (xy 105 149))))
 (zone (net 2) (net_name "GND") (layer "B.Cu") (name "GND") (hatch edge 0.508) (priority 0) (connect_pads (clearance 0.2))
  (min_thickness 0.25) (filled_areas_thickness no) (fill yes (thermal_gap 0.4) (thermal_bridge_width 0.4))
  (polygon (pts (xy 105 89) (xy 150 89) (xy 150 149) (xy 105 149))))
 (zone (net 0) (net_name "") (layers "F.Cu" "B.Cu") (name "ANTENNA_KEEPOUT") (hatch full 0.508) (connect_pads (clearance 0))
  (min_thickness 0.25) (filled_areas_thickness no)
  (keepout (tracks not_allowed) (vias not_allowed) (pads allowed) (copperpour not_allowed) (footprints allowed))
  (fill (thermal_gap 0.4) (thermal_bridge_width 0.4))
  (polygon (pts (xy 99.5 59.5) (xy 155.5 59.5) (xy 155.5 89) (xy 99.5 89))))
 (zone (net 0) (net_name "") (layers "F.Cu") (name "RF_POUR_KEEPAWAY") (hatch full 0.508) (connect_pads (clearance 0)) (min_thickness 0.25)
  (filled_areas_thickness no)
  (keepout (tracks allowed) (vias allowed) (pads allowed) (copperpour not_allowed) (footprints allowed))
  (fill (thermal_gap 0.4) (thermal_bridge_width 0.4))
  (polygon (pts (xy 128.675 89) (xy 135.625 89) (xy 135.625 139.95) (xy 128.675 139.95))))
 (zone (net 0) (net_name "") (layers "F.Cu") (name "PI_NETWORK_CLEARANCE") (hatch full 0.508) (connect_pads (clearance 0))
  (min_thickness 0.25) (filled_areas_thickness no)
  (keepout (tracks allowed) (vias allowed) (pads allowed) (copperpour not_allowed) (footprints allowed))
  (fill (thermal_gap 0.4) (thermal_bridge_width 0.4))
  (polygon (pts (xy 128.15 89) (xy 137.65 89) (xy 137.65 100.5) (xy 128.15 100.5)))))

